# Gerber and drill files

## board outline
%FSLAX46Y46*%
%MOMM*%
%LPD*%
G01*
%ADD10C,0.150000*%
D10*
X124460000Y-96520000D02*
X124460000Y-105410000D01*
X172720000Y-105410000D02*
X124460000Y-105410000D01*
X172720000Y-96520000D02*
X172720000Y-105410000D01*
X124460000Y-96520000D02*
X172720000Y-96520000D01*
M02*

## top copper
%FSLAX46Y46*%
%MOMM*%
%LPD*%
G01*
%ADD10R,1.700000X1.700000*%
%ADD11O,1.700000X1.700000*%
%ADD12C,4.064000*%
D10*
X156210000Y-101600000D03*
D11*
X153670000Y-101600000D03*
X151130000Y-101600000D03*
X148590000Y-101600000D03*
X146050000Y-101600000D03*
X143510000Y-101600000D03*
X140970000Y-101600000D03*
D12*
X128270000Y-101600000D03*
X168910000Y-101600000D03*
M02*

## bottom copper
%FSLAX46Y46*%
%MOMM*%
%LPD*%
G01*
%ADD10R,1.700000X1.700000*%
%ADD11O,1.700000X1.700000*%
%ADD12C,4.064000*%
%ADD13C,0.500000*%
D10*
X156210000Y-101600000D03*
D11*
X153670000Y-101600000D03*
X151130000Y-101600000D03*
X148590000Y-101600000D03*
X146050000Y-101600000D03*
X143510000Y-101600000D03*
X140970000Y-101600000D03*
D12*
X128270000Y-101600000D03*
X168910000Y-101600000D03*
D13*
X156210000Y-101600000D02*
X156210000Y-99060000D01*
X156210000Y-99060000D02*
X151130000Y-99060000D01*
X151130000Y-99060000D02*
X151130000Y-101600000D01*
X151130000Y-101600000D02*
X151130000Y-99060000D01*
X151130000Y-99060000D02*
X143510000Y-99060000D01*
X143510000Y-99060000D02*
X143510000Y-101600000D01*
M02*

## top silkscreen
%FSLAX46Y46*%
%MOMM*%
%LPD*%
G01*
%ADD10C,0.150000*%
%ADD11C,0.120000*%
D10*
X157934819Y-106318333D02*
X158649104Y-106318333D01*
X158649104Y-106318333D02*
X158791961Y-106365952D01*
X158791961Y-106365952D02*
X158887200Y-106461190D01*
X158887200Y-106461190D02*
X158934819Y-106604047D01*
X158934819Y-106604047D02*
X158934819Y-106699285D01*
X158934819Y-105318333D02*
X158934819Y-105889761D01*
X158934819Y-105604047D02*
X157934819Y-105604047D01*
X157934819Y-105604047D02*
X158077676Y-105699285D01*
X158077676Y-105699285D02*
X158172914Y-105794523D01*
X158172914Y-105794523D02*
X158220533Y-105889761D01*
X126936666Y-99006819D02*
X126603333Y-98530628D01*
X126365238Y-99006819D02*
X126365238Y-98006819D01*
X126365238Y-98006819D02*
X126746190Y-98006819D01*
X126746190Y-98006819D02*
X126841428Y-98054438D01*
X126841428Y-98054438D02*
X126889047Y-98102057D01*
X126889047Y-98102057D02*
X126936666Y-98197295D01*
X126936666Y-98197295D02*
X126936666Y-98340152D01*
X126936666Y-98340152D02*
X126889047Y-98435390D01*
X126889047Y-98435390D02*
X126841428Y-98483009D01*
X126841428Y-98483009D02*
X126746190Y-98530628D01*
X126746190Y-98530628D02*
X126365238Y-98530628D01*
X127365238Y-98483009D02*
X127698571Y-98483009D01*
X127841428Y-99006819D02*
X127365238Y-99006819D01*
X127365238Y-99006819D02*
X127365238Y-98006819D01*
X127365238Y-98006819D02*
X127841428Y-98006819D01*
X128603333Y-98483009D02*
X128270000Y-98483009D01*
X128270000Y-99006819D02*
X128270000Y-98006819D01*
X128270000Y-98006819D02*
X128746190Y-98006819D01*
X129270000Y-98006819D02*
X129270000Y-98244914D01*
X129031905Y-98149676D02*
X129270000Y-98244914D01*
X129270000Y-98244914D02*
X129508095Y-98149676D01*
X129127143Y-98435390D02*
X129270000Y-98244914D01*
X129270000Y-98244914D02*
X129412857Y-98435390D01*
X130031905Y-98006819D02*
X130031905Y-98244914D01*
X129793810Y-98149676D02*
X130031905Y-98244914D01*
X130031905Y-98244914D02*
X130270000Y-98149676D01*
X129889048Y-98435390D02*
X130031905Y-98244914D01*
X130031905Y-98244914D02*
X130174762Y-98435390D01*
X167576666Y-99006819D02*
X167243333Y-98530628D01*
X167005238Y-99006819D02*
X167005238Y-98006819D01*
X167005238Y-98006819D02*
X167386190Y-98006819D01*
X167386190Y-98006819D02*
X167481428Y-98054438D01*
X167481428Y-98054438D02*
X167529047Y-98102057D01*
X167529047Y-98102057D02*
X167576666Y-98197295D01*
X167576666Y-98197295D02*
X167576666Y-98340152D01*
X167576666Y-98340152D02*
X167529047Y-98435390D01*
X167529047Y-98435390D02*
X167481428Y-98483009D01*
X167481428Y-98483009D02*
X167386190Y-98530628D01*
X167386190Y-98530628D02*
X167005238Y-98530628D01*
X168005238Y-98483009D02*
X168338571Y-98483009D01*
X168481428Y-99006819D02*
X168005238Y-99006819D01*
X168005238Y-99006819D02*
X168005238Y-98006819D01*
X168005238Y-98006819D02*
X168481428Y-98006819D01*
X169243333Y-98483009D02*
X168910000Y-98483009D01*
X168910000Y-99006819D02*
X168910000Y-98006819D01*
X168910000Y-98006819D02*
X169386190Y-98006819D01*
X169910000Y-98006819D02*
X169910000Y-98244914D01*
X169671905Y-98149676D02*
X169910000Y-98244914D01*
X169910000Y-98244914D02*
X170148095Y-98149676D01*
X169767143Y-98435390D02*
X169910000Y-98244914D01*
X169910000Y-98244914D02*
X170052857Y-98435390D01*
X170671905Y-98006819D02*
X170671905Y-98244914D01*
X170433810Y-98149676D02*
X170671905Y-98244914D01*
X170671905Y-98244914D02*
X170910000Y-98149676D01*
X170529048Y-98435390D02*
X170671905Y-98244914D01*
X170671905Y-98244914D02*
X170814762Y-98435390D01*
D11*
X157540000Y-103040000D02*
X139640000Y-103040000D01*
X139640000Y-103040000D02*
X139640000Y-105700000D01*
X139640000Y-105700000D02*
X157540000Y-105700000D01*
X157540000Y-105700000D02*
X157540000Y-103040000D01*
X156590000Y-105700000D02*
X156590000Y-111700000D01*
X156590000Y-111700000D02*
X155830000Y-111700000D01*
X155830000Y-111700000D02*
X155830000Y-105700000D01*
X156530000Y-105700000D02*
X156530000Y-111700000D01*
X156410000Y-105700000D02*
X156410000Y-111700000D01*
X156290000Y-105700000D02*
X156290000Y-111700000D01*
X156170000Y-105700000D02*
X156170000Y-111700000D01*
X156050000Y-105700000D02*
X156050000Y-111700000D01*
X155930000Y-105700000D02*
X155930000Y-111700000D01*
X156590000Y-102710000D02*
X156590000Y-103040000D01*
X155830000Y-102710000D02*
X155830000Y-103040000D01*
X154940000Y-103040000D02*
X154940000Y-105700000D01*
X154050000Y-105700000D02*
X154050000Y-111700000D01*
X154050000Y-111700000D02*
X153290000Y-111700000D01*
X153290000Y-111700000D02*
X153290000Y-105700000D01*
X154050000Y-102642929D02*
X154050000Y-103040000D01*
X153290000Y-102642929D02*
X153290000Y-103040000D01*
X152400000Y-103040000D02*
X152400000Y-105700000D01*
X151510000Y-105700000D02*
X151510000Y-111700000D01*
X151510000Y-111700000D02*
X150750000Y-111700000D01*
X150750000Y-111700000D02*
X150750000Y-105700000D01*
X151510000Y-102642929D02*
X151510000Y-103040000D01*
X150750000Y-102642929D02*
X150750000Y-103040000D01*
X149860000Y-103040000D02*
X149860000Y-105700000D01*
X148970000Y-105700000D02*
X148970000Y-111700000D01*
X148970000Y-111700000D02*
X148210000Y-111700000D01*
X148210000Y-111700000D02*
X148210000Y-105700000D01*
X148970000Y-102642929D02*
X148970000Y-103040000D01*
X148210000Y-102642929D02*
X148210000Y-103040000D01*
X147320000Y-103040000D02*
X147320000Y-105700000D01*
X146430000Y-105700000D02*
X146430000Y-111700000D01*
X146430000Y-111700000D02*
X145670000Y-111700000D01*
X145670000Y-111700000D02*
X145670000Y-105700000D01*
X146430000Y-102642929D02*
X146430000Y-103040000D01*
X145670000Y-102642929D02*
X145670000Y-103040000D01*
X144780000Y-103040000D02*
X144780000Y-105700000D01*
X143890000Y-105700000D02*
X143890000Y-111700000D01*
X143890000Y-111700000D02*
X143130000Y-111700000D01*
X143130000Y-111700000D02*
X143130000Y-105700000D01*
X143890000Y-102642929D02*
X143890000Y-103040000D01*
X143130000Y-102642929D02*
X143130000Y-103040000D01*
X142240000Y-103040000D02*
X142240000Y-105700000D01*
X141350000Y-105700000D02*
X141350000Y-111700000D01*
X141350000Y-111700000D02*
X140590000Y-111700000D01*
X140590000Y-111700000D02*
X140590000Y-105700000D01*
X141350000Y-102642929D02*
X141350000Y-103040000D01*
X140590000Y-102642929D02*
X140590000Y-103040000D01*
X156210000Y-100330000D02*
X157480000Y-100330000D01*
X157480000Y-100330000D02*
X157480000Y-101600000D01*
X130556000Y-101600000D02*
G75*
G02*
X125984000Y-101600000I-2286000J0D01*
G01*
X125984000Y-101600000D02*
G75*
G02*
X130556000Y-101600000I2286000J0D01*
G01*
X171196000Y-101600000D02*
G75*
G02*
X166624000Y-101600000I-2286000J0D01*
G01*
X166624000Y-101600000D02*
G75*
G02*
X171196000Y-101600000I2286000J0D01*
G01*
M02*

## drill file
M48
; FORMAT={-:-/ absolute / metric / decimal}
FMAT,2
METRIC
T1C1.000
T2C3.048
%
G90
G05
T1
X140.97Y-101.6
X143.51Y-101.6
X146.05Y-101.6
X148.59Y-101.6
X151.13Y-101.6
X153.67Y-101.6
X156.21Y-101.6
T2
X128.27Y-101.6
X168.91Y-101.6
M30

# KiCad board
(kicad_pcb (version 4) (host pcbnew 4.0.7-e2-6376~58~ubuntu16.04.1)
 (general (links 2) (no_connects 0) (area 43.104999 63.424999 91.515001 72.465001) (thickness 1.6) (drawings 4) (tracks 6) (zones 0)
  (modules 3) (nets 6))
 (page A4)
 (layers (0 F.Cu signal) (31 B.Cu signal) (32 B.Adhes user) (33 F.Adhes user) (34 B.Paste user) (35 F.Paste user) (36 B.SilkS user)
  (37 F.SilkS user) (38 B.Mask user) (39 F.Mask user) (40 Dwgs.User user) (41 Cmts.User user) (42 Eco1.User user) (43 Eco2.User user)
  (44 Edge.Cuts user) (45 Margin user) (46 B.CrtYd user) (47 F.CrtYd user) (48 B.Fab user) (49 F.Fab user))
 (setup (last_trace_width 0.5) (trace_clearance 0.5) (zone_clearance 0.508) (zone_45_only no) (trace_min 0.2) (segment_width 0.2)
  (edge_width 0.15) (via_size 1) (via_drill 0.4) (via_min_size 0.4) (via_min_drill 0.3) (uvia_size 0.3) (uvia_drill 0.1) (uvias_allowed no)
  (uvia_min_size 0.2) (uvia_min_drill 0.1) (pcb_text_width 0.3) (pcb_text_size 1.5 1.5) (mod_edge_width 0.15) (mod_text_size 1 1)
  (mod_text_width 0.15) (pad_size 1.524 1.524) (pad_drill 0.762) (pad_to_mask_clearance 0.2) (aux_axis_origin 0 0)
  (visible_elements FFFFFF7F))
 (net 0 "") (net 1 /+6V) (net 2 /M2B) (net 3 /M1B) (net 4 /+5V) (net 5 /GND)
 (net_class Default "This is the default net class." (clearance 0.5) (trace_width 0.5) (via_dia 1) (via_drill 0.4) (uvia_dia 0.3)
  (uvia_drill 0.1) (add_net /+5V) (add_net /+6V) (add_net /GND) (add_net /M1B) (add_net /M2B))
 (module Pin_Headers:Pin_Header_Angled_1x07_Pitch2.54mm (layer F.Cu) (at 156.21 101.6 270)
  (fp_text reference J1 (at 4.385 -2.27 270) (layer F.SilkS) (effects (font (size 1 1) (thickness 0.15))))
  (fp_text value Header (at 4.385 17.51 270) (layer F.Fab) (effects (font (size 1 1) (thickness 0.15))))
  (fp_line (start 1.44 -1.33) (end 1.44 16.57) (layer F.SilkS) (width 0.12))
  (fp_line (start 1.44 16.57) (end 4.1 16.57) (layer F.SilkS) (width 0.12))
  (fp_line (start 4.1 16.57) (end 4.1 -1.33) (layer F.SilkS) (width 0.12))
  (fp_line (start 4.1 -1.33) (end 1.44 -1.33) (layer F.SilkS) (width 0.12))
  (fp_line (start 4.1 -0.38) (end 10.1 -0.38) (layer F.SilkS) (width 0.12))
  (fp_line (start 10.1 -0.38) (end 10.1 0.38) (layer F.SilkS) (width 0.12))
  (fp_line (start 10.1 0.38) (end 4.1 0.38) (layer F.SilkS) (width 0.12))
  (fp_line (start 4.1 -0.32) (end 10.1 -0.32) (layer F.SilkS) (width 0.12))
  (fp_line (start 4.1 -0.2) (end 10.1 -0.2) (layer F.SilkS) (width 0.12))
  (fp_line (start 4.1 -0.08) (end 10.1 -0.08) (layer F.SilkS) (width 0.12))
  (fp_line (start 4.1 0.04) (end 10.1 0.04) (layer F.SilkS) (width 0.12))
  (fp_line (start 4.1 0.16) (end 10.1 0.16) (layer F.SilkS) (width 0.12))
  (fp_line (start 4.1 0.28) (end 10.1 0.28) (layer F.SilkS) (width 0.12))
  (fp_line (start 1.11 -0.38) (end 1.44 -0.38) (layer F.SilkS) (width 0.12))
  (fp_line (start 1.11 0.38) (end 1.44 0.38) (layer F.SilkS) (width 0.12))
  (fp_line (start 1.44 1.27) (end 4.1 1.27) (layer F.SilkS) (width 0.12))
  (fp_line (start 4.1 2.16) (end 10.1 2.16) (layer F.SilkS) (width 0.12))
  (fp_line (start 10.1 2.16) (end 10.1 2.92) (layer F.SilkS) (width 0.12))
  (fp_line (start 10.1 2.92) (end 4.1 2.92) (layer F.SilkS) (width 0.12))
  (fp_line (start 1.042929 2.16) (end 1.44 2.16) (layer F.SilkS) (width 0.12))
  (fp_line (start 1.042929 2.92) (end 1.44 2.92) (layer F.SilkS) (width 0.12))
  (fp_line (start 1.44 3.81) (end 4.1 3.81) (layer F.SilkS) (width 0.12))
  (fp_line (start 4.1 4.7) (end 10.1 4.7) (layer F.SilkS) (width 0.12))
  (fp_line (start 10.1 4.7) (end 10.1 5.46) (layer F.SilkS) (width 0.12))
  (fp_line (start 10.1 5.46) (end 4.1 5.46) (layer F.SilkS) (width 0.12))
  (fp_line (start 1.042929 4.7) (end 1.44 4.7) (layer F.SilkS) (width 0.12))
  (fp_line (start 1.042929 5.46) (end 1.44 5.46) (layer F.SilkS) (width 0.12))
  (fp_line (start 1.44 6.35) (end 4.1 6.35) (layer F.SilkS) (width 0.12))
  (fp_line (start 4.1 7.24) (end 10.1 7.24) (layer F.SilkS) (width 0.12))
  (fp_line (start 10.1 7.24) (end 10.1 8) (layer F.SilkS) (width 0.12))
  (fp_line (start 10.1 8) (end 4.1 8) (layer F.SilkS) (width 0.12))
  (fp_line (start 1.042929 7.24) (end 1.44 7.24) (layer F.SilkS) (width 0.12))
  (fp_line (start 1.042929 8) (end 1.44 8) (layer F.SilkS) (width 0.12))
  (fp_line (start 1.44 8.89) (end 4.1 8.89) (layer F.SilkS) (width 0.12))
  (fp_line (start 4.1 9.78) (end 10.1 9.78) (layer F.SilkS) (width 0.12))
  (fp_line (start 10.1 9.78) (end 10.1 10.54) (layer F.SilkS) (width 0.12))
  (fp_line (start 10.1 10.54) (end 4.1 10.54) (layer F.SilkS) (width 0.12))
  (fp_line (start 1.042929 9.78) (end 1.44 9.78) (layer F.SilkS) (width 0.12))
  (fp_line (start 1.042929 10.54) (end 1.44 10.54) (layer F.SilkS) (width 0.12))
  (fp_line (start 1.44 11.43) (end 4.1 11.43) (layer F.SilkS) (width 0.12))
  (fp_line (start 4.1 12.32) (end 10.1 12.32) (layer F.SilkS) (width 0.12))
  (fp_line (start 10.1 12.32) (end 10.1 13.08) (layer F.SilkS) (width 0.12))
  (fp_line (start 10.1 13.08) (end 4.1 13.08) (layer F.SilkS) (width 0.12))
  (fp_line (start 1.042929 12.32) (end 1.44 12.32) (layer F.SilkS) (width 0.12))
  (fp_line (start 1.042929 13.08) (end 1.44 13.08) (layer F.SilkS) (width 0.12))
  (fp_line (start 1.44 13.97) (end 4.1 13.97) (layer F.SilkS) (width 0.12))
  (fp_line (start 4.1 14.86) (end 10.1 14.86) (layer F.SilkS) (width 0.12))
  (fp_line (start 10.1 14.86) (end 10.1 15.62) (layer F.SilkS) (width 0.12))
  (fp_line (start 10.1 15.62) (end 4.1 15.62) (layer F.SilkS) (width 0.12))
  (fp_line (start 1.042929 14.86) (end 1.44 14.86) (layer F.SilkS) (width 0.12))
  (fp_line (start 1.042929 15.62) (end 1.44 15.62) (layer F.SilkS) (width 0.12))
  (fp_line (start -1.27 0) (end -1.27 -1.27) (layer F.SilkS) (width 0.12))
  (fp_line (start -1.27 -1.27) (end 0 -1.27) (layer F.SilkS) (width 0.12))
  (pad 1 thru_hole rect (at 0 0 270) (size 1.7 1.7) (drill 1) (layers *.Cu *.Mask) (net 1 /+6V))
  (pad 2 thru_hole oval (at 0 2.54 270) (size 1.7 1.7) (drill 1) (layers *.Cu *.Mask) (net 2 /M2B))
  (pad 3 thru_hole oval (at 0 5.08 270) (size 1.7 1.7) (drill 1) (layers *.Cu *.Mask) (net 1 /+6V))
  (pad 4 thru_hole oval (at 0 7.62 270) (size 1.7 1.7) (drill 1) (layers *.Cu *.Mask) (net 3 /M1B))
  (pad 5 thru_hole oval (at 0 10.16 270) (size 1.7 1.7) (drill 1) (layers *.Cu *.Mask) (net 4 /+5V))
  (pad 6 thru_hole oval (at 0 12.7 270) (size 1.7 1.7) (drill 1) (layers *.Cu *.Mask) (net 1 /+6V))
  (pad 7 thru_hole oval (at 0 15.24 270) (size 1.7 1.7) (drill 1) (layers *.Cu *.Mask) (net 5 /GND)))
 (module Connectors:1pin (layer F.Cu) (at 128.27 101.6)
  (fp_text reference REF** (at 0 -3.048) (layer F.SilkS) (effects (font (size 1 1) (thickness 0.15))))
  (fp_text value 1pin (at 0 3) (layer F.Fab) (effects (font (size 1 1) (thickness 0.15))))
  (fp_circle (center 0 0) (end 0 -2.286) (layer F.SilkS) (width 0.12))
  (pad 1 thru_hole circle (at 0 0) (size 4.064 4.064) (drill 3.048) (layers *.Cu *.Mask)))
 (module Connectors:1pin (layer F.Cu) (at 168.91 101.6)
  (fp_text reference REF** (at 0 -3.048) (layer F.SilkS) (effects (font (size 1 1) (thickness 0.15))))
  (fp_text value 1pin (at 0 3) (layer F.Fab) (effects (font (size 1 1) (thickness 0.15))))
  (fp_circle (center 0 0) (end 0 -2.286) (layer F.SilkS) (width 0.12))
  (pad 1 thru_hole circle (at 0 0) (size 4.064 4.064) (drill 3.048) (layers *.Cu *.Mask)))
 (gr_line (start 124.46 96.52) (end 124.46 105.41) (angle 90) (layer Edge.Cuts) (width 0.15))
 (gr_line (start 172.72 105.41) (end 124.46 105.41) (angle 90) (layer Edge.Cuts) (width 0.15))
 (gr_line (start 172.72 96.52) (end 172.72 105.41) (angle 90) (layer Edge.Cuts) (width 0.15))
 (gr_line (start 124.46 96.52) (end 172.72 96.52) (angle 90) (layer Edge.Cuts) (width 0.15))
 (segment (start 156.21 101.6) (end 156.21 99.06) (width 0.5) (layer B.Cu) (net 1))
 (segment (start 156.21 99.06) (end 151.13 99.06) (width 0.5) (layer B.Cu) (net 1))
 (segment (start 151.13 99.06) (end 151.13 101.6) (width 0.5) (layer B.Cu) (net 1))
 (segment (start 151.13 101.6) (end 151.13 99.06) (width 0.5) (layer B.Cu) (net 1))
 (segment (start 151.13 99.06) (end 143.51 99.06) (width 0.5) (layer B.Cu) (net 1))
 (segment (start 143.51 99.06) (end 143.51 101.6) (width 0.5) (layer B.Cu) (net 1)))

